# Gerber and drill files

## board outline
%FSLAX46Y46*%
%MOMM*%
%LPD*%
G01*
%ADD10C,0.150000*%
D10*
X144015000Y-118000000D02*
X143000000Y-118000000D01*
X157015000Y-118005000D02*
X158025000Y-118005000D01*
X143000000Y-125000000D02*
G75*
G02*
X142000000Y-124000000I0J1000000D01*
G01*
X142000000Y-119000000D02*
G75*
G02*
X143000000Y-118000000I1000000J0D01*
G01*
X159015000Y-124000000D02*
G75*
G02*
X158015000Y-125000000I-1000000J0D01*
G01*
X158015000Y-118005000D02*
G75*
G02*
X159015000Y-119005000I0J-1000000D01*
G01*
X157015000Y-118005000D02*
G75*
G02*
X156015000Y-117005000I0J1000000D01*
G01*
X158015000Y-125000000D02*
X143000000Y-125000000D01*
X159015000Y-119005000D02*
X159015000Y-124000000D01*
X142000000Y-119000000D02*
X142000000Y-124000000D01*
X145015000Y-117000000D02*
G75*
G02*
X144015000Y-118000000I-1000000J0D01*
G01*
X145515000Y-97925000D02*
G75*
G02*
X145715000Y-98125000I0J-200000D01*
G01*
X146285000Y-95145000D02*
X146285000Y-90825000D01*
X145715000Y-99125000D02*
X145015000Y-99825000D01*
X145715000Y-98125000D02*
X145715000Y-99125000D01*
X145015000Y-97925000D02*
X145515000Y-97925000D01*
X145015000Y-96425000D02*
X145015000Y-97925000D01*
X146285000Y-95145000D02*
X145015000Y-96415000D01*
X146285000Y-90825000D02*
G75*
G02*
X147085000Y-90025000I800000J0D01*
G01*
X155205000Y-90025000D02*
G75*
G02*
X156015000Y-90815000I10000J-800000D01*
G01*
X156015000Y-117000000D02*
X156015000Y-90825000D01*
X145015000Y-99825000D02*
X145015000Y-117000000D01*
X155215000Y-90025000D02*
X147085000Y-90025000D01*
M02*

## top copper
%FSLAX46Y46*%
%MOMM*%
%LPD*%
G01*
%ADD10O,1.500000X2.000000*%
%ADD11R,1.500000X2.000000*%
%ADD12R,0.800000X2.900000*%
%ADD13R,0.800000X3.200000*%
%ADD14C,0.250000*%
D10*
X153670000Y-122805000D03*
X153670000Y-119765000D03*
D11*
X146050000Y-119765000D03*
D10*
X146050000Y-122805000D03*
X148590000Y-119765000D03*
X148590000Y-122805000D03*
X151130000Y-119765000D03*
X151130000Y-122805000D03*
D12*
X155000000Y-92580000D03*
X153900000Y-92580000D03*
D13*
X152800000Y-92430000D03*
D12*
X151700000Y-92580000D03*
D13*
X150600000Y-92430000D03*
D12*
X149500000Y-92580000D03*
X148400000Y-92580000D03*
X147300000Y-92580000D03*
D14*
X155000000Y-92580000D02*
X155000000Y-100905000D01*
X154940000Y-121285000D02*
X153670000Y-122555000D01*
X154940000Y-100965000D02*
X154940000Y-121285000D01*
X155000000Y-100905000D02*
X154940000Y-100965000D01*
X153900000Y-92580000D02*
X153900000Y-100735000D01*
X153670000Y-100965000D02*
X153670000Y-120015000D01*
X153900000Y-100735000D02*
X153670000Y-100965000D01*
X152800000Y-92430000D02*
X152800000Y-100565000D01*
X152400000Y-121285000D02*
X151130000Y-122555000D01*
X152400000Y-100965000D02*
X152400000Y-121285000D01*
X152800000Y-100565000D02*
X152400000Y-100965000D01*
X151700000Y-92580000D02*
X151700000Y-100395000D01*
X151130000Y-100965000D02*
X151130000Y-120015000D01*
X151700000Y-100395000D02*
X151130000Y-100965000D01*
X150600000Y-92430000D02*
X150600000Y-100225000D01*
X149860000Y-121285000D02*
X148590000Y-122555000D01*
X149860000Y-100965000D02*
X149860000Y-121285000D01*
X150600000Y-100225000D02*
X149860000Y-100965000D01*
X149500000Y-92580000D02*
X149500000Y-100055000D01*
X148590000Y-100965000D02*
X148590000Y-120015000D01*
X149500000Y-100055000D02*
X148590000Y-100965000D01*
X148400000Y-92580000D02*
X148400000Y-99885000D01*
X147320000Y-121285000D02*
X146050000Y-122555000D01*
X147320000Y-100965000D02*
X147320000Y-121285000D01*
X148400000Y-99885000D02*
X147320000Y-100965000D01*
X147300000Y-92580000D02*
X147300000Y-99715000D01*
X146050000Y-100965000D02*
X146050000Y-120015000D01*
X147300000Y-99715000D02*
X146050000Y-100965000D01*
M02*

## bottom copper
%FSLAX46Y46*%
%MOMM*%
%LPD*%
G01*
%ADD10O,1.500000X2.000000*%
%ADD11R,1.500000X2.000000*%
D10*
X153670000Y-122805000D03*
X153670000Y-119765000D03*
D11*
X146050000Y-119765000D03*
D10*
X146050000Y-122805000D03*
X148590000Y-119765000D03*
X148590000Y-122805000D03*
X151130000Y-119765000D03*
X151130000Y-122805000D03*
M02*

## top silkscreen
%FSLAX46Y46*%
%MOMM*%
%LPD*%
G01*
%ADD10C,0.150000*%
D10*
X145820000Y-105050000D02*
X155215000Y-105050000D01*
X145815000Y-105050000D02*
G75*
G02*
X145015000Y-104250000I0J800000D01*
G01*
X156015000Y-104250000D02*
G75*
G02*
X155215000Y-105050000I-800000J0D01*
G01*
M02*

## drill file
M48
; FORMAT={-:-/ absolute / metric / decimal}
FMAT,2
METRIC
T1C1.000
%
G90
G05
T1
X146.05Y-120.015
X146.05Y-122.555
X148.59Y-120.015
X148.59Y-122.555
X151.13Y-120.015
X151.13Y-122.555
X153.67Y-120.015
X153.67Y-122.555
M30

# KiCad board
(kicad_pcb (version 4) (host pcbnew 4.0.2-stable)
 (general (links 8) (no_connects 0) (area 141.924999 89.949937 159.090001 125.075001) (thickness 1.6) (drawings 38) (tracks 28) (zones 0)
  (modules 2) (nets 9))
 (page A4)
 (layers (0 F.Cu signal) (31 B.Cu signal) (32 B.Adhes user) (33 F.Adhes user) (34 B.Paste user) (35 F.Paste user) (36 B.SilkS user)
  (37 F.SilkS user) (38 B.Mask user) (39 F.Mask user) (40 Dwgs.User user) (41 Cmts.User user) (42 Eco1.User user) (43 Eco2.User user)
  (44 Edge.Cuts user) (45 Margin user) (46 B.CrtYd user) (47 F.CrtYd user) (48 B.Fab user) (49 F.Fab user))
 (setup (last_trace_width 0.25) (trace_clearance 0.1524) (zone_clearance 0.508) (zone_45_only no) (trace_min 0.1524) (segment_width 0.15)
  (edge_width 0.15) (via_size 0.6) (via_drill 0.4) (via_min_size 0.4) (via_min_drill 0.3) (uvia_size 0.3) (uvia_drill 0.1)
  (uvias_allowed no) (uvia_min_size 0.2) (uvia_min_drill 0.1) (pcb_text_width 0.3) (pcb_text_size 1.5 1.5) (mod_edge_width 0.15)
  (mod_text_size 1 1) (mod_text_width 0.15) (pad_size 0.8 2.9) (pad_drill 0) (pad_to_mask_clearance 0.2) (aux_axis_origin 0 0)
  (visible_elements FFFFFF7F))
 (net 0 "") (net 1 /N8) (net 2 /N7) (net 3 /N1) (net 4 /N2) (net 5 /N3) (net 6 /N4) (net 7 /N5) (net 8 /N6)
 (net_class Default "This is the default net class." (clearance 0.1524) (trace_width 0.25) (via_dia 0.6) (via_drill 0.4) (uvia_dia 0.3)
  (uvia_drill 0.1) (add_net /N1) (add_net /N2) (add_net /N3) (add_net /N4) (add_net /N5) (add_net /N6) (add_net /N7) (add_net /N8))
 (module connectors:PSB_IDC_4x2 (layer B.Cu) (at 149.86 121.285)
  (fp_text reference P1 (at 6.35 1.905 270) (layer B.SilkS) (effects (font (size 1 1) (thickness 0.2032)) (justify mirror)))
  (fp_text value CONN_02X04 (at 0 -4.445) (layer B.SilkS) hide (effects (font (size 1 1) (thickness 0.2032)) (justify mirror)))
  (pad 8 thru_hole oval (at 3.81 1.27) (size 1.5 2) (drill 1 (offset 0 0.25)) (layers *.Cu *.Mask B.SilkS) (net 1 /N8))
  (pad 7 thru_hole oval (at 3.81 -1.27) (size 1.5 2) (drill 1 (offset 0 -0.25)) (layers *.Cu *.Mask B.SilkS) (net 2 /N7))
  (pad 1 thru_hole rect (at -3.81 -1.27) (size 1.5 2) (drill 1 (offset 0 -0.25)) (layers *.Cu *.Mask B.SilkS) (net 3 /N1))
  (pad 2 thru_hole oval (at -3.81 1.27) (size 1.5 2) (drill 1 (offset 0 0.25)) (layers *.Cu *.Mask B.SilkS) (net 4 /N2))
  (pad 3 thru_hole oval (at -1.27 -1.27) (size 1.5 2) (drill 1 (offset 0 -0.25)) (layers *.Cu *.Mask B.SilkS) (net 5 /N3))
  (pad 4 thru_hole oval (at -1.27 1.27) (size 1.5 2) (drill 1 (offset 0 0.25)) (layers *.Cu *.Mask B.SilkS) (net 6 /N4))
  (pad 5 thru_hole oval (at 1.27 -1.27) (size 1.5 2) (drill 1 (offset 0 -0.25)) (layers *.Cu *.Mask B.SilkS) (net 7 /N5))
  (pad 6 thru_hole oval (at 1.27 1.27) (size 1.5 2) (drill 1 (offset 0 0.25)) (layers *.Cu *.Mask B.SilkS) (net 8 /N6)))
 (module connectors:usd (layer F.Cu) (at 147.3 92.58)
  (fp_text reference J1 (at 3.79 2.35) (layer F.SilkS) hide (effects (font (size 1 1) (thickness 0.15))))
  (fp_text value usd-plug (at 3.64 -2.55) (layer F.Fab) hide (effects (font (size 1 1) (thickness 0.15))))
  (pad 8 smd rect (at 7.7 0) (size 0.8 2.9) (layers F.Cu F.Paste F.Mask) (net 1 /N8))
  (pad 7 smd rect (at 6.6 0) (size 0.8 2.9) (layers F.Cu F.Paste F.Mask) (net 2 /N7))
  (pad 6 smd rect (at 5.5 -0.15) (size 0.8 3.2) (layers F.Cu F.Paste F.Mask) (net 8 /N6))
  (pad 5 smd rect (at 4.4 0) (size 0.8 2.9) (layers F.Cu F.Paste F.Mask) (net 7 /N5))
  (pad 4 smd rect (at 3.3 -0.15) (size 0.8 3.2) (layers F.Cu F.Paste F.Mask) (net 6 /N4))
  (pad 3 smd rect (at 2.2 0) (size 0.8 2.9) (layers F.Cu F.Paste F.Mask) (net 5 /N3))
  (pad 2 smd rect (at 1.1 0) (size 0.8 2.9) (layers F.Cu F.Paste F.Mask) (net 4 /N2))
  (pad 1 smd rect (at 0 0) (size 0.8 2.9) (layers F.Cu F.Paste F.Mask) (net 3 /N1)))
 (gr_line (start 144.015 118) (end 143 118) (angle 90) (layer Edge.Cuts) (width 0.15))
 (gr_line (start 157.015 118.005) (end 158.025 118.005) (angle 90) (layer Edge.Cuts) (width 0.15))
 (gr_arc (start 143 124) (end 143 125) (angle 90) (layer Edge.Cuts) (width 0.15))
 (gr_arc (start 143 119) (end 142 119) (angle 90) (layer Edge.Cuts) (width 0.15))
 (gr_arc (start 158.015 124) (end 159.015 124) (angle 90) (layer Edge.Cuts) (width 0.15))
 (gr_arc (start 158.015 119.005) (end 158.015 118.005) (angle 90) (layer Edge.Cuts) (width 0.15))
 (gr_arc (start 157.015 117.005) (end 157.015 118.005) (angle 90) (layer Edge.Cuts) (width 0.15))
 (gr_line (start 158.015 125) (end 143 125) (angle 90) (layer Edge.Cuts) (width 0.15))
 (gr_line (start 159.015 119.005) (end 159.015 124) (angle 90) (layer Edge.Cuts) (width 0.15))
 (gr_line (start 142 119) (end 142 124) (angle 90) (layer Edge.Cuts) (width 0.15))
 (gr_arc (start 144.015 117) (end 145.015 117) (angle 90) (layer Edge.Cuts) (width 0.15))
 (gr_line (start 145.82 105.05) (end 155.215 105.05) (angle 90) (layer F.SilkS) (width 0.15))
 (gr_arc (start 145.815 104.25) (end 145.815 105.05) (angle 90) (layer F.SilkS) (width 0.15))
 (gr_arc (start 155.215 104.25) (end 156.015 104.25) (angle 90) (layer F.SilkS) (width 0.15))
 (gr_arc (start 145.515 98.125) (end 145.715 98.125) (angle -90) (layer Edge.Cuts) (width 0.15))
 (gr_line (start 146.285 95.145) (end 146.285 90.825) (angle 90) (layer Edge.Cuts) (width 0.15))
 (gr_line (start 145.715 99.125) (end 145.015 99.825) (angle 90) (layer Edge.Cuts) (width 0.15))
 (gr_line (start 145.715 98.125) (end 145.715 99.125) (angle 90) (layer Edge.Cuts) (width 0.15))
 (gr_line (start 145.015 97.925) (end 145.515 97.925) (angle 90) (layer Edge.Cuts) (width 0.15))
 (gr_line (start 145.015 96.425) (end 145.015 97.925) (angle 90) (layer Edge.Cuts) (width 0.15))
 (gr_line (start 146.285 95.145) (end 145.015 96.415) (angle 90) (layer Edge.Cuts) (width 0.15))
 (gr_arc (start 147.085 90.825) (end 147.085 90.025) (angle -90) (layer Edge.Cuts) (width 0.15))
 (gr_arc (start 155.215 90.825) (end 156.015 90.815) (angle -90) (layer Edge.Cuts) (width 0.15))
 (gr_line (start 156.015 117) (end 156.015 90.825) (angle 90) (layer Edge.Cuts) (width 0.15))
 (gr_line (start 145.015 99.825) (end 145.015 117) (angle 90) (layer Edge.Cuts) (width 0.15))
 (gr_line (start 155.215 90.025) (end 147.085 90.025) (angle 90) (layer Edge.Cuts) (width 0.15))
 (segment (start 155 92.58) (end 155 100.905) (width 0.25) (layer F.Cu) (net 1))
 (segment (start 154.94 121.285) (end 153.67 122.555) (width 0.25) (layer F.Cu) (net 1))
 (segment (start 154.94 100.965) (end 154.94 121.285) (width 0.25) (layer F.Cu) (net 1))
 (segment (start 155 100.905) (end 154.94 100.965) (width 0.25) (layer F.Cu) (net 1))
 (segment (start 153.9 92.58) (end 153.9 100.735) (width 0.25) (layer F.Cu) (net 2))
 (segment (start 153.67 100.965) (end 153.67 120.015) (width 0.25) (layer F.Cu) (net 2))
 (segment (start 153.9 100.735) (end 153.67 100.965) (width 0.25) (layer F.Cu) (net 2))
 (segment (start 152.8 92.43) (end 152.8 100.565) (width 0.25) (layer F.Cu) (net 8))
 (segment (start 152.4 121.285) (end 151.13 122.555) (width 0.25) (layer F.Cu) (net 8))
 (segment (start 152.4 100.965) (end 152.4 121.285) (width 0.25) (layer F.Cu) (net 8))
 (segment (start 152.8 100.565) (end 152.4 100.965) (width 0.25) (layer F.Cu) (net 8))
 (segment (start 151.7 92.58) (end 151.7 100.395) (width 0.25) (layer F.Cu) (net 7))
 (segment (start 151.13 100.965) (end 151.13 120.015) (width 0.25) (layer F.Cu) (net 7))
 (segment (start 151.7 100.395) (end 151.13 100.965) (width 0.25) (layer F.Cu) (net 7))
 (segment (start 150.6 92.43) (end 150.6 100.225) (width 0.25) (layer F.Cu) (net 6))
 (segment (start 149.86 121.285) (end 148.59 122.555) (width 0.25) (layer F.Cu) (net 6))
 (segment (start 149.86 100.965) (end 149.86 121.285) (width 0.25) (layer F.Cu) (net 6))
 (segment (start 150.6 100.225) (end 149.86 100.965) (width 0.25) (layer F.Cu) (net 6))
 (segment (start 149.5 92.58) (end 149.5 100.055) (width 0.25) (layer F.Cu) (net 5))
 (segment (start 148.59 100.965) (end 148.59 120.015) (width 0.25) (layer F.Cu) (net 5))
 (segment (start 149.5 100.055) (end 148.59 100.965) (width 0.25) (layer F.Cu) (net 5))
 (segment (start 148.4 92.58) (end 148.4 99.885) (width 0.25) (layer F.Cu) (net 4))
 (segment (start 147.32 121.285) (end 146.05 122.555) (width 0.25) (layer F.Cu) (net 4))
 (segment (start 147.32 100.965) (end 147.32 121.285) (width 0.25) (layer F.Cu) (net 4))
 (segment (start 148.4 99.885) (end 147.32 100.965) (width 0.25) (layer F.Cu) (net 4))
 (segment (start 147.3 92.58) (end 147.3 99.715) (width 0.25) (layer F.Cu) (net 3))
 (segment (start 146.05 100.965) (end 146.05 120.015) (width 0.25) (layer F.Cu) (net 3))
 (segment (start 147.3 99.715) (end 146.05 100.965) (width 0.25) (layer F.Cu) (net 3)))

